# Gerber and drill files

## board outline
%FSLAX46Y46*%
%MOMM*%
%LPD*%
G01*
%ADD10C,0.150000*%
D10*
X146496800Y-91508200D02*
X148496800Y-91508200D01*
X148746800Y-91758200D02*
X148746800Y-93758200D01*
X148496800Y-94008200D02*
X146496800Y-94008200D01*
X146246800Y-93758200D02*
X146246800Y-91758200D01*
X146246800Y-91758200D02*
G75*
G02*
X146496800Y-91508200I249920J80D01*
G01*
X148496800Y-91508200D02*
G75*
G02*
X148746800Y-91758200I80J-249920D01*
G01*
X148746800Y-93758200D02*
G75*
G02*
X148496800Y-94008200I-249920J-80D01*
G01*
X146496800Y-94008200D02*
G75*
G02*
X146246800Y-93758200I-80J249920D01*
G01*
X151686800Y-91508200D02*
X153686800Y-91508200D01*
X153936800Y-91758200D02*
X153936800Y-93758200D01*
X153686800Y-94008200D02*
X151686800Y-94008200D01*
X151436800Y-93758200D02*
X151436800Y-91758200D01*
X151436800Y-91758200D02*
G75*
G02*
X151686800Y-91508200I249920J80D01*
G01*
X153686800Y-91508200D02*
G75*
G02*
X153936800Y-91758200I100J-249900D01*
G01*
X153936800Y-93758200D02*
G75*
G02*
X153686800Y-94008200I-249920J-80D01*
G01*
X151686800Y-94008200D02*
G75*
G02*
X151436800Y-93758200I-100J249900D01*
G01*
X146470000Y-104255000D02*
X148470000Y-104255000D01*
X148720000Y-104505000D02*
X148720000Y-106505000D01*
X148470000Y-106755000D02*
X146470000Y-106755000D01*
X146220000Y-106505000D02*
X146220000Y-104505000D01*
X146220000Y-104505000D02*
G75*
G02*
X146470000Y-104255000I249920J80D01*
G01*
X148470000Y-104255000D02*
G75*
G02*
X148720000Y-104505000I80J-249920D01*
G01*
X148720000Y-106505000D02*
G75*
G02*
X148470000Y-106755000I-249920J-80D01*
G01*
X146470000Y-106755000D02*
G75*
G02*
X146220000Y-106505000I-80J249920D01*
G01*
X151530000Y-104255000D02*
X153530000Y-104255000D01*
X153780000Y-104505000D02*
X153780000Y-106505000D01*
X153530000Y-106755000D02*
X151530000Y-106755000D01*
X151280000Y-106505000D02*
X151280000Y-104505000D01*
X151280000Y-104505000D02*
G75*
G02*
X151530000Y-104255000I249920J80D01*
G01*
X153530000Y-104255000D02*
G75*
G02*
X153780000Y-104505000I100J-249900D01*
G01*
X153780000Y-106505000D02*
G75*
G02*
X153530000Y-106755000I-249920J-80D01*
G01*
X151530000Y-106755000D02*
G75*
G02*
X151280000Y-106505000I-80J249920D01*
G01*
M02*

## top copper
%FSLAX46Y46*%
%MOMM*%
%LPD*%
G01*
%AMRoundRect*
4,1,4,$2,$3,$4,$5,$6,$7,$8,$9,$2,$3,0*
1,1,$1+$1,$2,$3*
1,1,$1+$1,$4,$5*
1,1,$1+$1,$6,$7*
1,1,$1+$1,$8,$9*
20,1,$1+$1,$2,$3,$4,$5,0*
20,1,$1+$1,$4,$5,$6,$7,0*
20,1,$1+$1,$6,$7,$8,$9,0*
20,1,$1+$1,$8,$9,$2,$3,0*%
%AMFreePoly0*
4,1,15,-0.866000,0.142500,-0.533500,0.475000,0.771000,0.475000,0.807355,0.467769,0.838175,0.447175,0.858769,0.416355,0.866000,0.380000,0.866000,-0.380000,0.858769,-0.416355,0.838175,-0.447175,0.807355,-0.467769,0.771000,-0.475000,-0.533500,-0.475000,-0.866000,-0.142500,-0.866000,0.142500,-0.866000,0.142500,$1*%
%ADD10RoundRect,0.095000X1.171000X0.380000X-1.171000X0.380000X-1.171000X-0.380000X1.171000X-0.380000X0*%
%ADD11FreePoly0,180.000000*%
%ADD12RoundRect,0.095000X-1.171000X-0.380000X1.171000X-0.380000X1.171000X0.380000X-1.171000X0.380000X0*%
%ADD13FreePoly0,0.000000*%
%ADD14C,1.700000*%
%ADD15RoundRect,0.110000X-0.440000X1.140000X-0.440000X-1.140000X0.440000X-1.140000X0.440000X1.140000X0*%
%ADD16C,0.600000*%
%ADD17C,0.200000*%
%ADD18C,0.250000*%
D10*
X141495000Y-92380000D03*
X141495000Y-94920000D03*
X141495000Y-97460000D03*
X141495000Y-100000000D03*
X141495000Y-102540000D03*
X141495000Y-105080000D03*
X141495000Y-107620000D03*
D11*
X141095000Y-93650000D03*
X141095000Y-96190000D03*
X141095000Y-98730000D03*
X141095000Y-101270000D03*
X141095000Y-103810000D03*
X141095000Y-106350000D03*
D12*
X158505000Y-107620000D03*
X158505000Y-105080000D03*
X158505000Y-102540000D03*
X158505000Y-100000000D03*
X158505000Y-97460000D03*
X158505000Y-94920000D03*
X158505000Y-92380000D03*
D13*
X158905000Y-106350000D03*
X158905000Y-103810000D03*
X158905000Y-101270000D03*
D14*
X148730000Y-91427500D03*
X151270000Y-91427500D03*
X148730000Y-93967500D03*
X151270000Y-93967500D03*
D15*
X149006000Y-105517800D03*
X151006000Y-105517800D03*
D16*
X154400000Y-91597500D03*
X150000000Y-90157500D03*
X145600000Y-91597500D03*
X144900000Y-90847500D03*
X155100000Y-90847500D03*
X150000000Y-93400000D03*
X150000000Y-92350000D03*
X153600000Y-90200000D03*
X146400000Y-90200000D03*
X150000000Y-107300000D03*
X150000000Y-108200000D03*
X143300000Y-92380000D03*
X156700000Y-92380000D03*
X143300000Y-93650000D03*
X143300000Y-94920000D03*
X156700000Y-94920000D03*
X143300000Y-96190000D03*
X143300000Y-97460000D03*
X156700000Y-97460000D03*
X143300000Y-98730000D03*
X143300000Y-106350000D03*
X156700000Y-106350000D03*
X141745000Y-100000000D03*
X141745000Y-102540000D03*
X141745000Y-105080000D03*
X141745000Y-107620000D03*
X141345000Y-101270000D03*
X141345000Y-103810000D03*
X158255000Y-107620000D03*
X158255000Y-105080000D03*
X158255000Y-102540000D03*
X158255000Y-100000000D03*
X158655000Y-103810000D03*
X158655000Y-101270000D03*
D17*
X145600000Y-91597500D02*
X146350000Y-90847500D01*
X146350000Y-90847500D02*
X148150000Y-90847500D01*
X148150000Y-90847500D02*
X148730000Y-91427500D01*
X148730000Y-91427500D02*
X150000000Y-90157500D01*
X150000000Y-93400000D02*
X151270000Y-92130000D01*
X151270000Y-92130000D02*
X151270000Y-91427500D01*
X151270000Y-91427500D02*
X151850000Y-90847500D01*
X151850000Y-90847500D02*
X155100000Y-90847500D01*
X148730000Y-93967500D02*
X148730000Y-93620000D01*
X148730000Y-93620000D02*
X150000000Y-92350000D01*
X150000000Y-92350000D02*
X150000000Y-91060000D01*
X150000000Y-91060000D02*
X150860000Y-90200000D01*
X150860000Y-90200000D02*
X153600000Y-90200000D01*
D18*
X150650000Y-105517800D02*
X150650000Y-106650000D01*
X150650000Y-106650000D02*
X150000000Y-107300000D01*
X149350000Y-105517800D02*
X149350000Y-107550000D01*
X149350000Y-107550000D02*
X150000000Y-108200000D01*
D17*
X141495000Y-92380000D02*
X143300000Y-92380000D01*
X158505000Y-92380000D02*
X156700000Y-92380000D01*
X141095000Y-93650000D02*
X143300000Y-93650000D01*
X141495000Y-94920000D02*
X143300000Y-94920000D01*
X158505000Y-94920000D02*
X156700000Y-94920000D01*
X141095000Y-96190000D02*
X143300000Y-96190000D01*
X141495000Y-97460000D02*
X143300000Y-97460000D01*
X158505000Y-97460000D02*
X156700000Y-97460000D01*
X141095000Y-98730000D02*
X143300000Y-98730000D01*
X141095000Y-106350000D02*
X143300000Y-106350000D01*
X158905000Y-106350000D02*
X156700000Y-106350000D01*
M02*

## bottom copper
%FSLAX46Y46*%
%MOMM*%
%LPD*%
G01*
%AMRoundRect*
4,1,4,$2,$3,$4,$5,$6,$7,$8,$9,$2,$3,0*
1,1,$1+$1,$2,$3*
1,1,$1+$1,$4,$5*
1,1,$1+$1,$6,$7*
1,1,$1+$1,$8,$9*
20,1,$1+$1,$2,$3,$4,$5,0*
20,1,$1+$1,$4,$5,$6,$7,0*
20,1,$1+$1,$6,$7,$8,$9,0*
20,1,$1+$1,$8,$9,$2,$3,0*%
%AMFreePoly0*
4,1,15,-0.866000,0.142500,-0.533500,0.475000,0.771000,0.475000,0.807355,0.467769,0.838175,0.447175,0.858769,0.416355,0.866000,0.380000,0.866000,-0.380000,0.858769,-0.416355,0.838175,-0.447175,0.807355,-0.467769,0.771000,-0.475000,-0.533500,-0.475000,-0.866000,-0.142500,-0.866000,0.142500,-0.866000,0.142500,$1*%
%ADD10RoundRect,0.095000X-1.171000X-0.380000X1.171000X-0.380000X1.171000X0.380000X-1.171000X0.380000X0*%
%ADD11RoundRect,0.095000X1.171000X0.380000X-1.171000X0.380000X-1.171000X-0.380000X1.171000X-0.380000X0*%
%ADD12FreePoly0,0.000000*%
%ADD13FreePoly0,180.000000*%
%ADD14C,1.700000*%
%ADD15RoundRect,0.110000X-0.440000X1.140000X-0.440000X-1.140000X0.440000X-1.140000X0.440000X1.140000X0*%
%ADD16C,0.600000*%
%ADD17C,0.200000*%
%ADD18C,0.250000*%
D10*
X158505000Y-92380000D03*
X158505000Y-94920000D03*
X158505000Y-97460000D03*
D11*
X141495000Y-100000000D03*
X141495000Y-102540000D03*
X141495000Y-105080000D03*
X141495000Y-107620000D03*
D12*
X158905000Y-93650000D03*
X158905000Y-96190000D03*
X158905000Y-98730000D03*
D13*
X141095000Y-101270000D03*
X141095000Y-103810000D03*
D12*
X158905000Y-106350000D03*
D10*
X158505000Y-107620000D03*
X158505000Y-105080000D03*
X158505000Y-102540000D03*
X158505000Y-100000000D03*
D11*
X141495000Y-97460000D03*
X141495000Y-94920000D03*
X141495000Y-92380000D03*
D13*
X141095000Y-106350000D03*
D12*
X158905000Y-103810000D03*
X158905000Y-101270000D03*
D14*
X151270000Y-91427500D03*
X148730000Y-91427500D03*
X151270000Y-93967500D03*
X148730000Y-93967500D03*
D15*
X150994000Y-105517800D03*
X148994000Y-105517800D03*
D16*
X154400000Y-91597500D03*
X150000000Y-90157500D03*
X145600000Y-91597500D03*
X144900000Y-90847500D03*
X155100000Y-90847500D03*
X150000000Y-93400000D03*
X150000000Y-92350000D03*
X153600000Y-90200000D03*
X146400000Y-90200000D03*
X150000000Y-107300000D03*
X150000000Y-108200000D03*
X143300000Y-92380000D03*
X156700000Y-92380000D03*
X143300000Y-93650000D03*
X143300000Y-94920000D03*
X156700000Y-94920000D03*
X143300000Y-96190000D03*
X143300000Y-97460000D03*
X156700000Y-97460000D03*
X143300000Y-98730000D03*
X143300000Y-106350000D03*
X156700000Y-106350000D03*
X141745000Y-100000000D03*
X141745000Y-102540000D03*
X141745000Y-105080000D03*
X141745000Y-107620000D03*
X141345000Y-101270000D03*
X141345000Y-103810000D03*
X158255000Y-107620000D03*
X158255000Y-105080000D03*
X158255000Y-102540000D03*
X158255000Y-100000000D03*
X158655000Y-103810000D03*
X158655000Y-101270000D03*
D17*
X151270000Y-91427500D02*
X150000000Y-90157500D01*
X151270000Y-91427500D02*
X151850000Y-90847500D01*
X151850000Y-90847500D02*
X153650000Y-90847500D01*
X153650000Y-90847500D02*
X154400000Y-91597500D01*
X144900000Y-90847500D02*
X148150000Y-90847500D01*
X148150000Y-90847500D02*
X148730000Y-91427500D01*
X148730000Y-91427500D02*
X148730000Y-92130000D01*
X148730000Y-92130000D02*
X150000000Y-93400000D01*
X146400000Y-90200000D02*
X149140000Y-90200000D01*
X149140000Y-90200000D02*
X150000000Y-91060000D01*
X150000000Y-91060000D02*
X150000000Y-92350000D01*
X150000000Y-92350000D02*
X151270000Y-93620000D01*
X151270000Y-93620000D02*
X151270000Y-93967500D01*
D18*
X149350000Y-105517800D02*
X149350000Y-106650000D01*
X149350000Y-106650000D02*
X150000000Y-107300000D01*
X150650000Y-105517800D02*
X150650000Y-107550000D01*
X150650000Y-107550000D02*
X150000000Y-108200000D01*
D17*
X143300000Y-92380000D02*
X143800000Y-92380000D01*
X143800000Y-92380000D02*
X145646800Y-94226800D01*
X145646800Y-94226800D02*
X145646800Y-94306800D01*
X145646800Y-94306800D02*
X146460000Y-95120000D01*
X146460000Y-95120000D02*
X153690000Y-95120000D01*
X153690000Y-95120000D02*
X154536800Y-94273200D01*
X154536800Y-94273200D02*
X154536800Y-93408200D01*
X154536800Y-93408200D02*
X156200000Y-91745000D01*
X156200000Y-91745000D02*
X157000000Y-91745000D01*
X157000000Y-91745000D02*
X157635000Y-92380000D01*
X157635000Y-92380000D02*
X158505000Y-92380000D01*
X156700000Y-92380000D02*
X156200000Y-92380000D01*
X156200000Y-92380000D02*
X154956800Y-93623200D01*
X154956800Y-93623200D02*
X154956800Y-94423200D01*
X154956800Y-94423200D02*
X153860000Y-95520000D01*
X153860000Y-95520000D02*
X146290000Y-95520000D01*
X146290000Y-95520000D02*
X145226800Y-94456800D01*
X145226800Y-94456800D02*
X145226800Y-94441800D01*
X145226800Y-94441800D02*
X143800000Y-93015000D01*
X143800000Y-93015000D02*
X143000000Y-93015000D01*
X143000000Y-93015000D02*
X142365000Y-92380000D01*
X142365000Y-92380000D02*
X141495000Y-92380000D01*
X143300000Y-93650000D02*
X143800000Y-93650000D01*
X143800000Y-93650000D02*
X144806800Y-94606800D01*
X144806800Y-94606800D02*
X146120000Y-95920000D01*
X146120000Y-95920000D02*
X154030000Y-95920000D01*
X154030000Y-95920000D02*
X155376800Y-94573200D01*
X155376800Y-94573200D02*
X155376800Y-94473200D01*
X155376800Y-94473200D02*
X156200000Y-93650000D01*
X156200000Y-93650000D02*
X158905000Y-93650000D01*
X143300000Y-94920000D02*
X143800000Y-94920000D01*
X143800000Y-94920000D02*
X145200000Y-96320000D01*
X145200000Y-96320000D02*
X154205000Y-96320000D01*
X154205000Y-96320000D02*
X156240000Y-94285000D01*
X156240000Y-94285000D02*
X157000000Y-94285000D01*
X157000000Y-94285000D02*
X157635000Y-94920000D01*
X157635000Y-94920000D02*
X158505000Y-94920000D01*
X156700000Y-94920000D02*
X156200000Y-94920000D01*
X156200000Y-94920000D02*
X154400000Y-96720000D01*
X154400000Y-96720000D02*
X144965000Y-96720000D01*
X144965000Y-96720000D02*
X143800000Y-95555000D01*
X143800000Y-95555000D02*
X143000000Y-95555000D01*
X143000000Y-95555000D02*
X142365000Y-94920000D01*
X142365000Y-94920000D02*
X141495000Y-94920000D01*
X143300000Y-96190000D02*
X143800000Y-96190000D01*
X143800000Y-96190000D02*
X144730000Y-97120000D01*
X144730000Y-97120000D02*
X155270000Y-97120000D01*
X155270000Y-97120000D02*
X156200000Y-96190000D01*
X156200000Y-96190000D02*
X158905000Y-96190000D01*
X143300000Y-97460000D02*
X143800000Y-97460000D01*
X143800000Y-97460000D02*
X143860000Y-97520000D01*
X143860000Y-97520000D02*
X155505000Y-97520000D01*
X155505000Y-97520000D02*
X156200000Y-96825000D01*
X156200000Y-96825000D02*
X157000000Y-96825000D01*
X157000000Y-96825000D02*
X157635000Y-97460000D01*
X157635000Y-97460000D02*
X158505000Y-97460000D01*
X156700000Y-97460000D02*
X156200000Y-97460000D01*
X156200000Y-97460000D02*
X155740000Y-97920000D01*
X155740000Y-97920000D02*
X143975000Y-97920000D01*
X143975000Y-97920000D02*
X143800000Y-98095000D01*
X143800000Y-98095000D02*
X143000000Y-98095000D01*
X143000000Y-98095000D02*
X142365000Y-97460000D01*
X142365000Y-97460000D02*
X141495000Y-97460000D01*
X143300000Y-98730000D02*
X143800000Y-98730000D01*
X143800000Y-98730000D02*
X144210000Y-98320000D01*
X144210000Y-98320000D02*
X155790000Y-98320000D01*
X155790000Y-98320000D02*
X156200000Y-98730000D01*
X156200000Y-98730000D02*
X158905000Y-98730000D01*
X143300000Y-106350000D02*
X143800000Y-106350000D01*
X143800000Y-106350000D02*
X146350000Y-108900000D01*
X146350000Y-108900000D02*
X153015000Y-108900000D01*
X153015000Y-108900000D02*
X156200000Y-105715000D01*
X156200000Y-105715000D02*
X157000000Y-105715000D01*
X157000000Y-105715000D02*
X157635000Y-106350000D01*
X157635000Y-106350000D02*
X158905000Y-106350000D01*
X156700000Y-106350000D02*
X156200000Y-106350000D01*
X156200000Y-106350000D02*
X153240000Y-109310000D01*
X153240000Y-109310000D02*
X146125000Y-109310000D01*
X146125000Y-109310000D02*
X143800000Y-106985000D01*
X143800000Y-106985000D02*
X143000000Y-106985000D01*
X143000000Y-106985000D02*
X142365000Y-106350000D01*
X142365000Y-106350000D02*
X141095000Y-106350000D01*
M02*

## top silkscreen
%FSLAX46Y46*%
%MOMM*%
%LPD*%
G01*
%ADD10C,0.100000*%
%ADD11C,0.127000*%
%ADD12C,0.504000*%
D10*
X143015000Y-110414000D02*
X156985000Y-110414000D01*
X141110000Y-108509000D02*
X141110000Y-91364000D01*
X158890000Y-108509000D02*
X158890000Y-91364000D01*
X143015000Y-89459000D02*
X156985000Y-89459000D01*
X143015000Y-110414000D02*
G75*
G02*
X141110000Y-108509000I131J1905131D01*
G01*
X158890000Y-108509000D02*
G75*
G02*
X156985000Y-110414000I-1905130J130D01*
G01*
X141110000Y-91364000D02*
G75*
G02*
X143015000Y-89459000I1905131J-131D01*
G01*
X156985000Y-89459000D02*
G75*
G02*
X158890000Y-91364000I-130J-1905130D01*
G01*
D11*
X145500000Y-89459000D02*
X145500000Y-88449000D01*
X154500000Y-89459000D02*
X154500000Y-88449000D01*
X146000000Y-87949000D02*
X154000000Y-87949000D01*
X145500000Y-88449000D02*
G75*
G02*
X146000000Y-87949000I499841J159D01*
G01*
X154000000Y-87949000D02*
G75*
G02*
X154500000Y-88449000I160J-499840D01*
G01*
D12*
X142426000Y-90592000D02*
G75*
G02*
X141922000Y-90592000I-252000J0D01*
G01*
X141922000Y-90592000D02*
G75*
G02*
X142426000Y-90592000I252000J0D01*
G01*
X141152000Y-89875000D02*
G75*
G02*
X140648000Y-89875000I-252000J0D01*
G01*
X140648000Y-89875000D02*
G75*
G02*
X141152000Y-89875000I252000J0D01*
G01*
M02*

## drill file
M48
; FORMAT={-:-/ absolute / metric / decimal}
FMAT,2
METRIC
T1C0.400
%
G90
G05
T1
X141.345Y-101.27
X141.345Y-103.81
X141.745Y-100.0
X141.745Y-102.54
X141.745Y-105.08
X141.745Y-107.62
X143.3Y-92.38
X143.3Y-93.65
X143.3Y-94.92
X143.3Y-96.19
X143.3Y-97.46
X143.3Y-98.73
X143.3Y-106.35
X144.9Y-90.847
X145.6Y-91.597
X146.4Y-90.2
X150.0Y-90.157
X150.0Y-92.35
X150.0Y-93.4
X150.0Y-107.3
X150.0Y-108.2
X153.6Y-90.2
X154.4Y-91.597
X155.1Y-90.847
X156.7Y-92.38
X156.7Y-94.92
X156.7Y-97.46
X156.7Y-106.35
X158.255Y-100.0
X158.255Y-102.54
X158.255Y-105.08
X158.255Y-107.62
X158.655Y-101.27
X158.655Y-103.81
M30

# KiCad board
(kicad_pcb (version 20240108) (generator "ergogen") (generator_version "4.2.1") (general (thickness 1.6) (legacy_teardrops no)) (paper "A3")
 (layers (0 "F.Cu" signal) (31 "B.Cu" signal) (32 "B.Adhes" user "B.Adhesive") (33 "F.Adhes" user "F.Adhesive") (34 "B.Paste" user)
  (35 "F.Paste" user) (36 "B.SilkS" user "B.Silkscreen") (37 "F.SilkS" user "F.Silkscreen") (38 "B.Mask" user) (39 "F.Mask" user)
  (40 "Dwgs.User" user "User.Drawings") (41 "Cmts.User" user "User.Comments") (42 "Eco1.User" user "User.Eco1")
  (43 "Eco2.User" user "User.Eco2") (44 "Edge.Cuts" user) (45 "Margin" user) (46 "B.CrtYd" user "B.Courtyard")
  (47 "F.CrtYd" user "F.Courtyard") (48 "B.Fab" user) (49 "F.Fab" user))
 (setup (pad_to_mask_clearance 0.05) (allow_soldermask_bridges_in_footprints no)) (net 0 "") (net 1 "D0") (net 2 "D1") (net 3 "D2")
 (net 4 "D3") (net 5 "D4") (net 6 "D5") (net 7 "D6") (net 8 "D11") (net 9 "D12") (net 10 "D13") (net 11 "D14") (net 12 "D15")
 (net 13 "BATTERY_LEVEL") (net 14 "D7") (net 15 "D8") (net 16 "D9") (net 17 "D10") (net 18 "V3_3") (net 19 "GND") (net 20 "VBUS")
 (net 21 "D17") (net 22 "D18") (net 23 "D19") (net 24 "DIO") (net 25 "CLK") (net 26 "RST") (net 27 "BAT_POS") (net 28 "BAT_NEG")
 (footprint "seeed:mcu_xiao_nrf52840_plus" (layer "F.Cu") (at 150 100 0)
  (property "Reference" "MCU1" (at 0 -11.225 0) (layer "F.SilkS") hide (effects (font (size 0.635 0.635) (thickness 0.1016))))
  (pad "1" smd roundrect (at -8.505 -7.62 180) (size 2.532 0.95) (layers "F.Cu" "F.Mask" "F.Paste") (roundrect_rratio 0.1) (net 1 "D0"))
  (pad "2" smd roundrect (at -8.505 -5.08 180) (size 2.532 0.95) (layers "F.Cu" "F.Mask" "F.Paste") (roundrect_rratio 0.1) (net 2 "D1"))
  (pad "3" smd roundrect (at -8.505 -2.54 180) (size 2.532 0.95) (layers "F.Cu" "F.Mask" "F.Paste") (roundrect_rratio 0.1) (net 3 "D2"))
  (pad "4" smd roundrect (at -8.505 0 180) (size 2.532 0.95) (layers "F.Cu" "F.Mask" "F.Paste") (roundrect_rratio 0.1) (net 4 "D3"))
  (pad "5" smd roundrect (at -8.505 2.54 180) (size 2.532 0.95) (layers "F.Cu" "F.Mask" "F.Paste") (roundrect_rratio 0.1) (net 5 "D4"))
  (pad "6" smd roundrect (at -8.505 5.08 180) (size 2.532 0.95) (layers "F.Cu" "F.Mask" "F.Paste") (roundrect_rratio 0.1) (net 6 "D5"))
  (pad "7" smd roundrect (at -8.505 7.62 180) (size 2.532 0.95) (layers "F.Cu" "F.Mask" "F.Paste") (roundrect_rratio 0.1) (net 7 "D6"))
  (pad "15" smd roundrect (at -8.905 -6.35 180) (size 1.732 0.95) (layers "F.Cu" "F.Mask" "F.Paste") (roundrect_rratio 0.1)
   (chamfer_ratio 0.35) (chamfer top_left bottom_left) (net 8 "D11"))
  (pad "16" smd roundrect (at -8.905 -3.81 180) (size 1.732 0.95) (layers "F.Cu" "F.Mask" "F.Paste") (roundrect_rratio 0.1)
   (chamfer_ratio 0.35) (chamfer top_left bottom_left) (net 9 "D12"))
  (pad "17" smd roundrect (at -8.905 -1.27 180) (size 1.732 0.95) (layers "F.Cu" "F.Mask" "F.Paste") (roundrect_rratio 0.1)
   (chamfer_ratio 0.35) (chamfer top_left bottom_left) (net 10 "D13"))
  (pad "18" smd roundrect (at -8.905 1.27 180) (size 1.732 0.95) (layers "F.Cu" "F.Mask" "F.Paste") (roundrect_rratio 0.1)
   (chamfer_ratio 0.35) (chamfer top_left bottom_left) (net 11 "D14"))
  (pad "19" smd roundrect (at -8.905 3.81 180) (size 1.732 0.95) (layers "F.Cu" "F.Mask" "F.Paste") (roundrect_rratio 0.1)
   (chamfer_ratio 0.35) (chamfer top_left bottom_left) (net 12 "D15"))
  (pad "20" smd roundrect (at -8.905 6.35 180) (size 1.732 0.95) (layers "F.Cu" "F.Mask" "F.Paste") (roundrect_rratio 0.1)
   (chamfer_ratio 0.35) (chamfer top_left bottom_left) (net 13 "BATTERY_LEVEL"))
  (pad "8" smd roundrect (at 8.505 7.62 0) (size 2.532 0.95) (layers "F.Cu" "F.Mask" "F.Paste") (roundrect_rratio 0.1) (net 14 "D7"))
  (pad "9" smd roundrect (at 8.505 5.08 0) (size 2.532 0.95) (layers "F.Cu" "F.Mask" "F.Paste") (roundrect_rratio 0.1) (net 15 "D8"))
  (pad "10" smd roundrect (at 8.505 2.54 0) (size 2.532 0.95) (layers "F.Cu" "F.Mask" "F.Paste") (roundrect_rratio 0.1) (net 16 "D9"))
  (pad "11" smd roundrect (at 8.505 0 0) (size 2.532 0.95) (layers "F.Cu" "F.Mask" "F.Paste") (roundrect_rratio 0.1) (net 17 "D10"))
  (pad "12" smd roundrect (at 8.505 -2.54 0) (size 2.532 0.95) (layers "F.Cu" "F.Mask" "F.Paste") (roundrect_rratio 0.1) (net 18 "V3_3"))
  (pad "13" smd roundrect (at 8.505 -5.08 0) (size 2.532 0.95) (layers "F.Cu" "F.Mask" "F.Paste") (roundrect_rratio 0.1) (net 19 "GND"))
  (pad "14" smd roundrect (at 8.505 -7.62 0) (size 2.532 0.95) (layers "F.Cu" "F.Mask" "F.Paste") (roundrect_rratio 0.1) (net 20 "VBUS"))
  (pad "21" smd roundrect (at 8.905 6.35 0) (size 1.732 0.95) (layers "F.Cu" "F.Mask" "F.Paste") (roundrect_rratio 0.1) (chamfer_ratio 0.35)
   (chamfer top_left bottom_left) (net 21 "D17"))
  (pad "22" smd roundrect (at 8.905 3.81 0) (size 1.732 0.95) (layers "F.Cu" "F.Mask" "F.Paste") (roundrect_rratio 0.1) (chamfer_ratio 0.35)
   (chamfer top_left bottom_left) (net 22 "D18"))
  (pad "23" smd roundrect (at 8.905 1.27 0) (size 1.732 0.95) (layers "F.Cu" "F.Mask" "F.Paste") (roundrect_rratio 0.1) (chamfer_ratio 0.35)
   (chamfer top_left bottom_left) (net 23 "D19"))
  (pad "24" smd circle (at -1.27 -8.5725 0) (size 1.7 1.7) (layers "F.Cu" "F.Mask" "F.Paste") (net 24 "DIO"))
  (pad "25" smd circle (at 1.27 -8.5725 0) (size 1.7 1.7) (layers "F.Cu" "F.Mask" "F.Paste") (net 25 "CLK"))
  (pad "26" smd circle (at -1.27 -6.0325 0) (size 1.7 1.7) (layers "F.Cu" "F.Mask" "F.Paste") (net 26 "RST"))
  (pad "27" smd circle (at 1.27 -6.0325 0) (size 1.7 1.7) (layers "F.Cu" "F.Mask" "F.Paste") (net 19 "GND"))
  (pad "28" smd roundrect (at -0.994 5.5178 270) (size 2.5 1.1) (layers "F.Cu" "F.Mask" "F.Paste") (roundrect_rratio 0.1) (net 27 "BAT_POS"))
  (pad "29" smd roundrect (at 1.006 5.5178 270) (size 2.5 1.1) (layers "F.Cu" "F.Mask" "F.Paste") (roundrect_rratio 0.1) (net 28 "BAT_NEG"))
  (fp_line (start -6.985 10.414) (end 6.985 10.414) (stroke (width 0.1) (type solid)) (layer "F.SilkS"))
  (fp_line (start -8.89 8.509) (end -8.89 -8.636) (stroke (width 0.1) (type solid)) (layer "F.SilkS"))
  (fp_line (start 8.89 8.509) (end 8.89 -8.636) (stroke (width 0.1) (type solid)) (layer "F.SilkS"))
  (fp_line (start -6.985 -10.541) (end 6.985 -10.541) (stroke (width 0.1) (type solid)) (layer "F.SilkS"))
  (fp_arc (start -6.985 10.414) (mid -8.332 9.856) (end -8.89 8.509) (stroke (width 0.1) (type solid)) (layer "F.SilkS"))
  (fp_arc (start 8.89 8.509) (mid 8.332 9.856) (end 6.985 10.414) (stroke (width 0.1) (type solid)) (layer "F.SilkS"))
  (fp_arc (start -8.89 -8.636) (mid -8.332 -9.983) (end -6.985 -10.541) (stroke (width 0.1) (type solid)) (layer "F.SilkS"))
  (fp_arc (start 6.985 -10.541) (mid 8.332 -9.983) (end 8.89 -8.636) (stroke (width 0.1) (type solid)) (layer "F.SilkS"))
  (fp_line (start -4.5 -10.541) (end -4.5 -11.551) (stroke (width 0.127) (type solid)) (layer "F.SilkS"))
  (fp_line (start 4.5 -10.541) (end 4.5 -11.551) (stroke (width 0.127) (type solid)) (layer "F.SilkS"))
  (fp_line (start -4 -12.051) (end 4 -12.051) (stroke (width 0.127) (type solid)) (layer "F.SilkS"))
  (fp_arc (start -4.5 -11.551) (mid -4.3536 -11.9046) (end -4 -12.051) (stroke (width 0.127) (type solid)) (layer "F.SilkS"))
  (fp_arc (start 4 -12.051) (mid 4.3536 -11.9046) (end 4.5 -11.551) (stroke (width 0.127) (type solid)) (layer "F.SilkS"))
  (fp_circle (center -7.826 -9.408) (end -7.826 -9.662) (stroke (width 0.5) (type solid)) (fill yes) (layer "F.SilkS"))
  (fp_circle (center -9.1 -10.125) (end -9.1 -10.379) (stroke (width 0.5) (type solid)) (fill yes) (layer "F.SilkS"))
  (pad "1" smd roundrect (at 8.505 -7.62 0) (size 2.532 0.95) (layers "B.Cu" "B.Mask" "B.Paste") (roundrect_rratio 0.1) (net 1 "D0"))
  (pad "2" smd roundrect (at 8.505 -5.08 0) (size 2.532 0.95) (layers "B.Cu" "B.Mask" "B.Paste") (roundrect_rratio 0.1) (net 2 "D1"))
  (pad "3" smd roundrect (at 8.505 -2.54 0) (size 2.532 0.95) (layers "B.Cu" "B.Mask" "B.Paste") (roundrect_rratio 0.1) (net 3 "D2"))
  (pad "4" smd roundrect (at -8.505 0 180) (size 2.532 0.95) (layers "B.Cu" "B.Mask" "B.Paste") (roundrect_rratio 0.1) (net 4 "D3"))
  (pad "5" smd roundrect (at -8.505 2.54 180) (size 2.532 0.95) (layers "B.Cu" "B.Mask" "B.Paste") (roundrect_rratio 0.1) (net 5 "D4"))
  (pad "6" smd roundrect (at -8.505 5.08 180) (size 2.532 0.95) (layers "B.Cu" "B.Mask" "B.Paste") (roundrect_rratio 0.1) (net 6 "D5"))
  (pad "7" smd roundrect (at -8.505 7.62 180) (size 2.532 0.95) (layers "B.Cu" "B.Mask" "B.Paste") (roundrect_rratio 0.1) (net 7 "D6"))
  (pad "15" smd roundrect (at 8.905 -6.35 0) (size 1.732 0.95) (layers "B.Cu" "B.Mask" "B.Paste") (roundrect_rratio 0.1)
   (chamfer_ratio 0.35) (chamfer top_left bottom_left) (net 8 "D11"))
  (pad "16" smd roundrect (at 8.905 -3.81 0) (size 1.732 0.95) (layers "B.Cu" "B.Mask" "B.Paste") (roundrect_rratio 0.1)
   (chamfer_ratio 0.35) (chamfer top_left bottom_left) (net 9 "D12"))
  (pad "17" smd roundrect (at 8.905 -1.27 0) (size 1.732 0.95) (layers "B.Cu" "B.Mask" "B.Paste") (roundrect_rratio 0.1)
   (chamfer_ratio 0.35) (chamfer top_left bottom_left) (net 10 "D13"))
  (pad "18" smd roundrect (at -8.905 1.27 180) (size 1.732 0.95) (layers "B.Cu" "B.Mask" "B.Paste") (roundrect_rratio 0.1)
   (chamfer_ratio 0.35) (chamfer top_left bottom_left) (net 11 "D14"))
  (pad "19" smd roundrect (at -8.905 3.81 180) (size 1.732 0.95) (layers "B.Cu" "B.Mask" "B.Paste") (roundrect_rratio 0.1)
   (chamfer_ratio 0.35) (chamfer top_left bottom_left) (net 12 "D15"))
  (pad "20" smd roundrect (at 8.905 6.35 0) (size 1.732 0.95) (layers "B.Cu" "B.Mask" "B.Paste") (roundrect_rratio 0.1) (chamfer_ratio 0.35)
   (chamfer top_left bottom_left) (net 13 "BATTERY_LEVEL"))
  (pad "8" smd roundrect (at 8.505 7.62 0) (size 2.532 0.95) (layers "B.Cu" "B.Mask" "B.Paste") (roundrect_rratio 0.1) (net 14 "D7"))
  (pad "9" smd roundrect (at 8.505 5.08 0) (size 2.532 0.95) (layers "B.Cu" "B.Mask" "B.Paste") (roundrect_rratio 0.1) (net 15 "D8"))
  (pad "10" smd roundrect (at 8.505 2.54 0) (size 2.532 0.95) (layers "B.Cu" "B.Mask" "B.Paste") (roundrect_rratio 0.1) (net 16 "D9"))
  (pad "11" smd roundrect (at 8.505 0 0) (size 2.532 0.95) (layers "B.Cu" "B.Mask" "B.Paste") (roundrect_rratio 0.1) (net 17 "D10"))
  (pad "12" smd roundrect (at -8.505 -2.54 180) (size 2.532 0.95) (layers "B.Cu" "B.Mask" "B.Paste") (roundrect_rratio 0.1) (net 18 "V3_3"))
  (pad "13" smd roundrect (at -8.505 -5.08 180) (size 2.532 0.95) (layers "B.Cu" "B.Mask" "B.Paste") (roundrect_rratio 0.1) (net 19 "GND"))
  (pad "14" smd roundrect (at -8.505 -7.62 180) (size 2.532 0.95) (layers "B.Cu" "B.Mask" "B.Paste") (roundrect_rratio 0.1) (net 20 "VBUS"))
  (pad "21" smd roundrect (at -8.905 6.35 180) (size 1.732 0.95) (layers "B.Cu" "B.Mask" "B.Paste") (roundrect_rratio 0.1)
   (chamfer_ratio 0.35) (chamfer top_left bottom_left) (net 21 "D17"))
  (pad "22" smd roundrect (at 8.905 3.81 0) (size 1.732 0.95) (layers "B.Cu" "B.Mask" "B.Paste") (roundrect_rratio 0.1) (chamfer_ratio 0.35)
   (chamfer top_left bottom_left) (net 22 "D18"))
  (pad "23" smd roundrect (at 8.905 1.27 0) (size 1.732 0.95) (layers "B.Cu" "B.Mask" "B.Paste") (roundrect_rratio 0.1) (chamfer_ratio 0.35)
   (chamfer top_left bottom_left) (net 23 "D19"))
  (pad "24" smd circle (at 1.27 -8.5725 0) (size 1.7 1.7) (layers "B.Cu" "B.Mask" "B.Paste") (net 24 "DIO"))
  (pad "25" smd circle (at -1.27 -8.5725 0) (size 1.7 1.7) (layers "B.Cu" "B.Mask" "B.Paste") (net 25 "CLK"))
  (pad "26" smd circle (at 1.27 -6.0325 0) (size 1.7 1.7) (layers "B.Cu" "B.Mask" "B.Paste") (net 26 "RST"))
  (pad "27" smd circle (at -1.27 -6.0325 0) (size 1.7 1.7) (layers "B.Cu" "B.Mask" "B.Paste") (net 19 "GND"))
  (pad "28" smd roundrect (at 0.994 5.5178 270) (size 2.5 1.1) (layers "B.Cu" "B.Mask" "B.Paste") (roundrect_rratio 0.1) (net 27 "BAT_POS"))
  (pad "29" smd roundrect (at -1.006 5.5178 270) (size 2.5 1.1) (layers "B.Cu" "B.Mask" "B.Paste") (roundrect_rratio 0.1) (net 28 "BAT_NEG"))
  (fp_line (start -3.5032 -8.4918) (end -1.5032 -8.4918) (stroke (width 0.15) (type default)) (layer "Edge.Cuts"))
  (fp_line (start -1.2532 -8.2418) (end -1.2532 -6.2418) (stroke (width 0.15) (type default)) (layer "Edge.Cuts"))
  (fp_line (start -1.5032 -5.9918) (end -3.5032 -5.9918) (stroke (width 0.15) (type default)) (layer "Edge.Cuts"))
  (fp_line (start -3.7532 -6.2418) (end -3.7532 -8.2418) (stroke (width 0.15) (type default)) (layer "Edge.Cuts"))
  (fp_arc (start -3.7532 -8.2418) (mid -3.68 -8.4186) (end -3.5032 -8.4918) (stroke (width 0.15) (type default)) (layer "Edge.Cuts"))
  (fp_arc (start -1.5032 -8.4918) (mid -1.3264 -8.4186) (end -1.2532 -8.2418) (stroke (width 0.15) (type default)) (layer "Edge.Cuts"))
  (fp_arc (start -1.2532 -6.2418) (mid -1.3264 -6.065) (end -1.5032 -5.9918) (stroke (width 0.15) (type default)) (layer "Edge.Cuts"))
  (fp_arc (start -3.5032 -5.9918) (mid -3.68 -6.065) (end -3.7532 -6.2418) (stroke (width 0.15) (type default)) (layer "Edge.Cuts"))
  (fp_line (start 1.6868 -8.4918) (end 3.6868 -8.4918) (stroke (width 0.15) (type default)) (layer "Edge.Cuts"))
  (fp_line (start 3.9368 -8.2418) (end 3.9368 -6.2418) (stroke (width 0.15) (type default)) (layer "Edge.Cuts"))
  (fp_line (start 3.6868 -5.9918) (end 1.6868 -5.9918) (stroke (width 0.15) (type default)) (layer "Edge.Cuts"))
  (fp_line (start 1.4368 -6.2418) (end 1.4368 -8.2418) (stroke (width 0.15) (type default)) (layer "Edge.Cuts"))
  (fp_arc (start 1.4368 -8.2418) (mid 1.51 -8.4186) (end 1.6868 -8.4918) (stroke (width 0.15) (type default)) (layer "Edge.Cuts"))
  (fp_arc (start 3.6868 -8.4918) (mid 3.8636 -8.4186) (end 3.9368 -8.2418) (stroke (width 0.15) (type default)) (layer "Edge.Cuts"))
  (fp_arc (start 3.9368 -6.2418) (mid 3.8636 -6.065) (end 3.6868 -5.9918) (stroke (width 0.15) (type default)) (layer "Edge.Cuts"))
  (fp_arc (start 1.6868 -5.9918) (mid 1.51 -6.065) (end 1.4368 -6.2418) (stroke (width 0.15) (type default)) (layer "Edge.Cuts"))
  (fp_line (start -3.53 4.255) (end -1.53 4.255) (stroke (width 0.15) (type default)) (layer "Edge.Cuts"))
  (fp_line (start -1.28 4.505) (end -1.28 6.505) (stroke (width 0.15) (type default)) (layer "Edge.Cuts"))
  (fp_line (start -1.53 6.755) (end -3.53 6.755) (stroke (width 0.15) (type default)) (layer "Edge.Cuts"))
  (fp_line (start -3.78 6.505) (end -3.78 4.505) (stroke (width 0.15) (type default)) (layer "Edge.Cuts"))
  (fp_arc (start -3.78 4.505) (mid -3.7068 4.3282) (end -3.53 4.255) (stroke (width 0.15) (type default)) (layer "Edge.Cuts"))
  (fp_arc (start -1.53 4.255) (mid -1.3532 4.3282) (end -1.28 4.505) (stroke (width 0.15) (type default)) (layer "Edge.Cuts"))
  (fp_arc (start -1.28 6.505) (mid -1.3532 6.6818) (end -1.53 6.755) (stroke (width 0.15) (type default)) (layer "Edge.Cuts"))
  (fp_arc (start -3.53 6.755) (mid -3.7068 6.6818) (end -3.78 6.505) (stroke (width 0.15) (type default)) (layer "Edge.Cuts"))
  (fp_line (start 1.53 4.255) (end 3.53 4.255) (stroke (width 0.15) (type default)) (layer "Edge.Cuts"))
  (fp_line (start 3.78 4.505) (end 3.78 6.505) (stroke (width 0.15) (type default)) (layer "Edge.Cuts"))
  (fp_line (start 3.53 6.755) (end 1.53 6.755) (stroke (width 0.15) (type default)) (layer "Edge.Cuts"))
  (fp_line (start 1.28 6.505) (end 1.28 4.505) (stroke (width 0.15) (type default)) (layer "Edge.Cuts"))
  (fp_arc (start 1.28 4.505) (mid 1.3532 4.3282) (end 1.53 4.255) (stroke (width 0.15) (type default)) (layer "Edge.Cuts"))
  (fp_arc (start 3.53 4.255) (mid 3.7068 4.3282) (end 3.78 4.505) (stroke (width 0.15) (type default)) (layer "Edge.Cuts"))
  (fp_arc (start 3.78 6.505) (mid 3.7068 6.6818) (end 3.53 6.755) (stroke (width 0.15) (type default)) (layer "Edge.Cuts"))
  (fp_arc (start 1.53 6.755) (mid 1.3532 6.6818) (end 1.28 6.505) (stroke (width 0.15) (type default)) (layer "Edge.Cuts")))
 (segment (start 151.27 91.4275) (end 150 90.1575) (width 0.2) (layer "B.Cu") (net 24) (locked no))
 (segment (start 151.27 91.4275) (end 151.85 90.8475) (width 0.2) (layer "B.Cu") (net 24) (locked no))
 (segment (start 151.85 90.8475) (end 153.65 90.8475) (width 0.2) (layer "B.Cu") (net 24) (locked no))
 (segment (start 153.65 90.8475) (end 154.4 91.5975) (width 0.2) (layer "B.Cu") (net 24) (locked no))
 (segment (start 145.6 91.5975) (end 146.35 90.8475) (width 0.2) (layer "F.Cu") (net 24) (locked no))
 (segment (start 146.35 90.8475) (end 148.15 90.8475) (width 0.2) (layer "F.Cu") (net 24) (locked no))
 (segment (start 148.15 90.8475) (end 148.73 91.4275) (width 0.2) (layer "F.Cu") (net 24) (locked no))
 (segment (start 148.73 91.4275) (end 150 90.1575) (width 0.2) (layer "F.Cu") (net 24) (locked no))
 (via (at 154.4 91.5975) (size 0.6) (drill 0.4) (layers "F.Cu" "B.Cu") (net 24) (locked no))
 (via (at 150 90.1575) (size 0.6) (drill 0.4) (layers "F.Cu" "B.Cu") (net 24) (locked no))
 (via (at 145.6 91.5975) (size 0.6) (drill 0.4) (layers "F.Cu" "B.Cu") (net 24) (locked no))
 (segment (start 144.9 90.8475) (end 148.15 90.8475) (width 0.2) (layer "B.Cu") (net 25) (locked no))
 (segment (start 148.15 90.8475) (end 148.73 91.4275) (width 0.2) (layer "B.Cu") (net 25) (locked no))
 (segment (start 148.73 91.4275) (end 148.73 92.13) (width 0.2) (layer "B.Cu") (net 25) (locked no))
 (segment (start 148.73 92.13) (end 150 93.4) (width 0.2) (layer "B.Cu") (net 25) (locked no))
 (segment (start 150 93.4) (end 151.27 92.13) (width 0.2) (layer "F.Cu") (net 25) (locked no))
 (segment (start 151.27 92.13) (end 151.27 91.4275) (width 0.2) (layer "F.Cu") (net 25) (locked no))
 (segment (start 151.27 91.4275) (end 151.85 90.8475) (width 0.2) (layer "F.Cu") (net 25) (locked no))
 (segment (start 151.85 90.8475) (end 155.1 90.8475) (width 0.2) (layer "F.Cu") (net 25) (locked no))
 (via (at 144.9 90.8475) (size 0.6) (drill 0.4) (layers "F.Cu" "B.Cu") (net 25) (locked no))
 (via (at 155.1 90.8475) (size 0.6) (drill 0.4) (layers "F.Cu" "B.Cu") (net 25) (locked no))
 (via (at 150 93.4) (size 0.6) (drill 0.4) (layers "F.Cu" "B.Cu") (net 25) (locked no))
 (segment (start 146.4 90.2) (end 149.14 90.2) (width 0.2) (layer "B.Cu") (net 26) (locked no))
 (segment (start 149.14 90.2) (end 150 91.06) (width 0.2) (layer "B.Cu") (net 26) (locked no))
 (segment (start 150 91.06) (end 150 92.35) (width 0.2) (layer "B.Cu") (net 26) (locked no))
 (segment (start 150 92.35) (end 151.27 93.62) (width 0.2) (layer "B.Cu") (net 26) (locked no))
 (segment (start 151.27 93.62) (end 151.27 93.9675) (width 0.2) (layer "B.Cu") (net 26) (locked no))
 (segment (start 148.73 93.9675) (end 148.73 93.62) (width 0.2) (layer "F.Cu") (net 26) (locked no))
 (segment (start 148.73 93.62) (end 150 92.35) (width 0.2) (layer "F.Cu") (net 26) (locked no))
 (segment (start 150 92.35) (end 150 91.06) (width 0.2) (layer "F.Cu") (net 26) (locked no))
 (segment (start 150 91.06) (end 150.86 90.2) (width 0.2) (layer "F.Cu") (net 26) (locked no))
 (segment (start 150.86 90.2) (end 153.6 90.2) (width 0.2) (layer "F.Cu") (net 26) (locked no))
 (via (at 150 92.35) (size 0.6) (drill 0.4) (layers "F.Cu" "B.Cu") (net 26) (locked no))
 (via (at 153.6 90.2) (size 0.6) (drill 0.4) (layers "F.Cu" "B.Cu") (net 26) (locked no))
 (via (at 146.4 90.2) (size 0.6) (drill 0.4) (layers "F.Cu" "B.Cu") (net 26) (locked no))
 (segment (start 149.35 105.5178) (end 149.35 106.65) (width 0.25) (layer "B.Cu") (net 28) (locked no))
 (segment (start 149.35 106.65) (end 150 107.3) (width 0.25) (layer "B.Cu") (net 28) (locked no))
 (segment (start 150.65 105.5178) (end 150.65 106.65) (width 0.25) (layer "F.Cu") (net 28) (locked no))
 (segment (start 150.65 106.65) (end 150 107.3) (width 0.25) (layer "F.Cu") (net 28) (locked no))
 (segment (start 150.65 105.5178) (end 150.65 107.55) (width 0.25) (layer "B.Cu") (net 27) (locked no))
 (segment (start 150.65 107.55) (end 150 108.2) (width 0.25) (layer "B.Cu") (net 27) (locked no))
 (segment (start 149.35 105.5178) (end 149.35 107.55) (width 0.25) (layer "F.Cu") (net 27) (locked no))
 (segment (start 149.35 107.55) (end 150 108.2) (width 0.25) (layer "F.Cu") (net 27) (locked no))
 (via (at 150 107.3) (size 0.6) (drill 0.4) (layers "F.Cu" "B.Cu") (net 28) (locked no))
 (via (at 150 108.2) (size 0.6) (drill 0.4) (layers "F.Cu" "B.Cu") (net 27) (locked no))
 (segment (start 141.495 92.38) (end 143.3 92.38) (width 0.2) (layer "F.Cu") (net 1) (locked no))
 (segment (start 143.3 92.38) (end 143.8 92.38) (width 0.2) (layer "B.Cu") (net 1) (locked no))
 (segment (start 143.8 92.38) (end 145.6468 94.2268) (width 0.2) (layer "B.Cu") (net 1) (locked no))
 (segment (start 145.6468 94.2268) (end 145.6468 94.3068) (width 0.2) (layer "B.Cu") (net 1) (locked no))
 (segment (start 145.6468 94.3068) (end 146.46 95.12) (width 0.2) (layer "B.Cu") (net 1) (locked no))
 (segment (start 146.46 95.12) (end 153.69 95.12) (width 0.2) (layer "B.Cu") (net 1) (locked no))
 (segment (start 153.69 95.12) (end 154.5368 94.2732) (width 0.2) (layer "B.Cu") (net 1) (locked no))
 (segment (start 154.5368 94.2732) (end 154.5368 93.4082) (width 0.2) (layer "B.Cu") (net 1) (locked no))
 (segment (start 154.5368 93.4082) (end 156.2 91.745) (width 0.2) (layer "B.Cu") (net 1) (locked no))
 (segment (start 156.2 91.745) (end 157 91.745) (width 0.2) (layer "B.Cu") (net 1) (locked no))
 (segment (start 157 91.745) (end 157.635 92.38) (width 0.2) (layer "B.Cu") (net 1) (locked no))
 (segment (start 157.635 92.38) (end 158.505 92.38) (width 0.2) (layer "B.Cu") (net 1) (locked no))
 (segment (start 158.505 92.38) (end 156.7 92.38) (width 0.2) (layer "F.Cu") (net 20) (locked no))
 (segment (start 156.7 92.38) (end 156.2 92.38) (width 0.2) (layer "B.Cu") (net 20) (locked no))
 (segment (start 156.2 92.38) (end 154.9568 93.6232) (width 0.2) (layer "B.Cu") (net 20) (locked no))
 (segment (start 154.9568 93.6232) (end 154.9568 94.4232) (width 0.2) (layer "B.Cu") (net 20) (locked no))
 (segment (start 154.9568 94.4232) (end 153.86 95.52) (width 0.2) (layer "B.Cu") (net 20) (locked no))
 (segment (start 153.86 95.52) (end 146.29 95.52) (width 0.2) (layer "B.Cu") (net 20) (locked no))
 (segment (start 146.29 95.52) (end 145.2268 94.4568) (width 0.2) (layer "B.Cu") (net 20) (locked no))
 (segment (start 145.2268 94.4568) (end 145.2268 94.4418) (width 0.2) (layer "B.Cu") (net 20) (locked no))
 (segment (start 145.2268 94.4418) (end 143.8 93.015) (width 0.2) (layer "B.Cu") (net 20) (locked no))
 (segment (start 143.8 93.015) (end 143 93.015) (width 0.2) (layer "B.Cu") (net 20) (locked no))
 (segment (start 143 93.015) (end 142.365 92.38) (width 0.2) (layer "B.Cu") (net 20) (locked no))
 (segment (start 142.365 92.38) (end 141.495 92.38) (width 0.2) (layer "B.Cu") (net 20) (locked no))
 (segment (start 141.095 93.65) (end 143.3 93.65) (width 0.2) (layer "F.Cu") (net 8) (locked no))
 (segment (start 143.3 93.65) (end 143.8 93.65) (width 0.2) (layer "B.Cu") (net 8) (locked no))
 (segment (start 143.8 93.65) (end 144.8068 94.60679999999999) (width 0.2) (layer "B.Cu") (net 8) (locked no))
 (segment (start 144.8068 94.60679999999999) (end 146.12 95.92) (width 0.2) (layer "B.Cu") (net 8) (locked no))
 (segment (start 146.12 95.92) (end 154.03 95.92) (width 0.2) (layer "B.Cu") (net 8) (locked no))
 (segment (start 154.03 95.92) (end 155.3768 94.5732) (width 0.2) (layer "B.Cu") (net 8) (locked no))
 (segment (start 155.3768 94.5732) (end 155.3768 94.4732) (width 0.2) (layer "B.Cu") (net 8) (locked no))
 (segment (start 155.3768 94.4732) (end 156.2 93.65) (width 0.2) (layer "B.Cu") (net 8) (locked no))
 (segment (start 156.2 93.65) (end 158.905 93.65) (width 0.2) (layer "B.Cu") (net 8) (locked no))
 (segment (start 141.495 94.92) (end 143.3 94.92) (width 0.2) (layer "F.Cu") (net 2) (locked no))
 (segment (start 143.3 94.92) (end 143.8 94.92) (width 0.2) (layer "B.Cu") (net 2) (locked no))
 (segment (start 143.8 94.92) (end 145.2 96.32) (width 0.2) (layer "B.Cu") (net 2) (locked no))
 (segment (start 145.2 96.32) (end 154.205 96.32) (width 0.2) (layer "B.Cu") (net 2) (locked no))
 (segment (start 154.205 96.32) (end 156.24 94.285) (width 0.2) (layer "B.Cu") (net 2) (locked no))
 (segment (start 156.24 94.285) (end 157 94.285) (width 0.2) (layer "B.Cu") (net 2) (locked no))
 (segment (start 157 94.285) (end 157.635 94.92) (width 0.2) (layer "B.Cu") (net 2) (locked no))
 (segment (start 157.635 94.92) (end 158.505 94.92) (width 0.2) (layer "B.Cu") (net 2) (locked no))
 (segment (start 158.505 94.92) (end 156.7 94.92) (width 0.2) (layer "F.Cu") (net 19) (locked no))
 (segment (start 156.7 94.92) (end 156.2 94.92) (width 0.2) (layer "B.Cu") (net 19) (locked no))
 (segment (start 156.2 94.92) (end 154.4 96.72) (width 0.2) (layer "B.Cu") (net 19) (locked no))
 (segment (start 154.4 96.72) (end 144.965 96.72) (width 0.2) (layer "B.Cu") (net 19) (locked no))
 (segment (start 144.965 96.72) (end 143.8 95.555) (width 0.2) (layer "B.Cu") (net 19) (locked no))
 (segment (start 143.8 95.555) (end 143 95.555) (width 0.2) (layer "B.Cu") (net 19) (locked no))
 (segment (start 143 95.555) (end 142.365 94.92) (width 0.2) (layer "B.Cu") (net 19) (locked no))
 (segment (start 142.365 94.92) (end 141.495 94.92) (width 0.2) (layer "B.Cu") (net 19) (locked no))
 (segment (start 141.095 96.19) (end 143.3 96.19) (width 0.2) (layer "F.Cu") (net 9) (locked no))
 (segment (start 143.3 96.19) (end 143.8 96.19) (width 0.2) (layer "B.Cu") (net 9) (locked no))
 (segment (start 143.8 96.19) (end 144.73 97.12) (width 0.2) (layer "B.Cu") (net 9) (locked no))
 (segment (start 144.73 97.12) (end 155.27 97.12) (width 0.2) (layer "B.Cu") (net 9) (locked no))
 (segment (start 155.27 97.12) (end 156.2 96.19) (width 0.2) (layer "B.Cu") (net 9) (locked no))
 (segment (start 156.2 96.19) (end 158.905 96.19) (width 0.2) (layer "B.Cu") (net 9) (locked no))
 (segment (start 141.495 97.46) (end 143.3 97.46) (width 0.2) (layer "F.Cu") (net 3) (locked no))
 (segment (start 143.3 97.46) (end 143.8 97.46) (width 0.2) (layer "B.Cu") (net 3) (locked no))
 (segment (start 143.8 97.46) (end 143.86 97.52) (width 0.2) (layer "B.Cu") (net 3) (locked no))
 (segment (start 143.86 97.52) (end 155.505 97.52) (width 0.2) (layer "B.Cu") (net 3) (locked no))
 (segment (start 155.505 97.52) (end 156.2 96.825) (width 0.2) (layer "B.Cu") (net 3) (locked no))
 (segment (start 156.2 96.825) (end 157 96.825) (width 0.2) (layer "B.Cu") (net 3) (locked no))
 (segment (start 157 96.825) (end 157.635 97.46) (width 0.2) (layer "B.Cu") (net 3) (locked no))
 (segment (start 157.635 97.46) (end 158.505 97.46) (width 0.2) (layer "B.Cu") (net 3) (locked no))
 (segment (start 158.505 97.46) (end 156.7 97.46) (width 0.2) (layer "F.Cu") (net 18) (locked no))
 (segment (start 156.7 97.46) (end 156.2 97.46) (width 0.2) (layer "B.Cu") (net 18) (locked no))
 (segment (start 156.2 97.46) (end 155.74 97.92) (width 0.2) (layer "B.Cu") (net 18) (locked no))
 (segment (start 155.74 97.92) (end 143.975 97.92) (width 0.2) (layer "B.Cu") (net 18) (locked no))
 (segment (start 143.975 97.92) (end 143.8 98.095) (width 0.2) (layer "B.Cu") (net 18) (locked no))
 (segment (start 143.8 98.095) (end 143 98.095) (width 0.2) (layer "B.Cu") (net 18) (locked no))
 (segment (start 143 98.095) (end 142.365 97.46) (width 0.2) (layer "B.Cu") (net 18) (locked no))
 (segment (start 142.365 97.46) (end 141.495 97.46) (width 0.2) (layer "B.Cu") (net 18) (locked no))
 (segment (start 141.095 98.73) (end 143.3 98.73) (width 0.2) (layer "F.Cu") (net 10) (locked no))
 (segment (start 143.3 98.73) (end 143.8 98.73) (width 0.2) (layer "B.Cu") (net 10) (locked no))
 (segment (start 143.8 98.73) (end 144.21 98.32) (width 0.2) (layer "B.Cu") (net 10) (locked no))
 (segment (start 144.21 98.32) (end 155.79 98.32) (width 0.2) (layer "B.Cu") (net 10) (locked no))
 (segment (start 155.79 98.32) (end 156.2 98.73) (width 0.2) (layer "B.Cu") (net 10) (locked no))
 (segment (start 156.2 98.73) (end 158.905 98.73) (width 0.2) (layer "B.Cu") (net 10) (locked no))
 (segment (start 141.095 106.35) (end 143.3 106.35) (width 0.2) (layer "F.Cu") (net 13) (locked no))
 (segment (start 143.3 106.35) (end 143.8 106.35) (width 0.2) (layer "B.Cu") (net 13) (locked no))
 (segment (start 143.8 106.35) (end 146.35 108.9) (width 0.2) (layer "B.Cu") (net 13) (locked no))
 (segment (start 146.35 108.9) (end 153.015 108.9) (width 0.2) (layer "B.Cu") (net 13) (locked no))
 (segment (start 153.015 108.9) (end 156.2 105.715) (width 0.2) (layer "B.Cu") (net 13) (locked no))
 (segment (start 156.2 105.715) (end 157 105.715) (width 0.2) (layer "B.Cu") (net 13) (locked no))
 (segment (start 157 105.715) (end 157.635 106.35) (width 0.2) (layer "B.Cu") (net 13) (locked no))
 (segment (start 157.635 106.35) (end 158.905 106.35) (width 0.2) (layer "B.Cu") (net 13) (locked no))
 (segment (start 158.905 106.35) (end 156.7 106.35) (width 0.2) (layer "F.Cu") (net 21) (locked no))
 (segment (start 156.7 106.35) (end 156.2 106.35) (width 0.2) (layer "B.Cu") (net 21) (locked no))
 (segment (start 156.2 106.35) (end 153.24 109.31) (width 0.2) (layer "B.Cu") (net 21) (locked no))
 (segment (start 153.24 109.31) (end 146.125 109.31) (width 0.2) (layer "B.Cu") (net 21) (locked no))
 (segment (start 146.125 109.31) (end 143.8 106.985) (width 0.2) (layer "B.Cu") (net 21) (locked no))
 (segment (start 143.8 106.985) (end 143 106.985) (width 0.2) (layer "B.Cu") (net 21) (locked no))
 (segment (start 143 106.985) (end 142.365 106.35) (width 0.2) (layer "B.Cu") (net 21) (locked no))
 (segment (start 142.365 106.35) (end 141.095 106.35) (width 0.2) (layer "B.Cu") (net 21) (locked no))
 (via (at 143.3 92.38) (size 0.6) (drill 0.4) (layers "F.Cu" "B.Cu") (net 1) (locked no))
 (via (at 156.7 92.38) (size 0.6) (drill 0.4) (layers "F.Cu" "B.Cu") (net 20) (locked no))
 (via (at 143.3 93.65) (size 0.6) (drill 0.4) (layers "F.Cu" "B.Cu") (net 8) (locked no))
 (via (at 143.3 94.92) (size 0.6) (drill 0.4) (layers "F.Cu" "B.Cu") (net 2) (locked no))
 (via (at 156.7 94.92) (size 0.6) (drill 0.4) (layers "F.Cu" "B.Cu") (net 19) (locked no))
 (via (at 143.3 96.19) (size 0.6) (drill 0.4) (layers "F.Cu" "B.Cu") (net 9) (locked no))
 (via (at 143.3 97.46) (size 0.6) (drill 0.4) (layers "F.Cu" "B.Cu") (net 3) (locked no))
 (via (at 156.7 97.46) (size 0.6) (drill 0.4) (layers "F.Cu" "B.Cu") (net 18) (locked no))
 (via (at 143.3 98.73) (size 0.6) (drill 0.4) (layers "F.Cu" "B.Cu") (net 10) (locked no))
 (via (at 143.3 106.35) (size 0.6) (drill 0.4) (layers "F.Cu" "B.Cu") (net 13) (locked no))
 (via (at 156.7 106.35) (size 0.6) (drill 0.4) (layers "F.Cu" "B.Cu") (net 21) (locked no))
 (via (at 141.745 100) (size 0.6) (drill 0.4) (layers "F.Cu" "B.Cu") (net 4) (locked no))
 (via (at 141.745 102.54) (size 0.6) (drill 0.4) (layers "F.Cu" "B.Cu") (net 5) (locked no))
 (via (at 141.745 105.08) (size 0.6) (drill 0.4) (layers "F.Cu" "B.Cu") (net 6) (locked no))
 (via (at 141.745 107.62) (size 0.6) (drill 0.4) (layers "F.Cu" "B.Cu") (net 7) (locked no))
 (via (at 141.345 101.27) (size 0.6) (drill 0.4) (layers "F.Cu" "B.Cu") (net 11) (locked no))
 (via (at 141.345 103.81) (size 0.6) (drill 0.4) (layers "F.Cu" "B.Cu") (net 12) (locked no))
 (via (at 158.255 107.62) (size 0.6) (drill 0.4) (layers "F.Cu" "B.Cu") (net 14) (locked no))
 (via (at 158.255 105.08) (size 0.6) (drill 0.4) (layers "F.Cu" "B.Cu") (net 15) (locked no))
 (via (at 158.255 102.54) (size 0.6) (drill 0.4) (layers "F.Cu" "B.Cu") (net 16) (locked no))
 (via (at 158.255 100) (size 0.6) (drill 0.4) (layers "F.Cu" "B.Cu") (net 17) (locked no))
 (via (at 158.655 103.81) (size 0.6) (drill 0.4) (layers "F.Cu" "B.Cu") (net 22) (locked no))
 (via (at 158.655 101.27) (size 0.6) (drill 0.4) (layers "F.Cu" "B.Cu") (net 23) (locked no))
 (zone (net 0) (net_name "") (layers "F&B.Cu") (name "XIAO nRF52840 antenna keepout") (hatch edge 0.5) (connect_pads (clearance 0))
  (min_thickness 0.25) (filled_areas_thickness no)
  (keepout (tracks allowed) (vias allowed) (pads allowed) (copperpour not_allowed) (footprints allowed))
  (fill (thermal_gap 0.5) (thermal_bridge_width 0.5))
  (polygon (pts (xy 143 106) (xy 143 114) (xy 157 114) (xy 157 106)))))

